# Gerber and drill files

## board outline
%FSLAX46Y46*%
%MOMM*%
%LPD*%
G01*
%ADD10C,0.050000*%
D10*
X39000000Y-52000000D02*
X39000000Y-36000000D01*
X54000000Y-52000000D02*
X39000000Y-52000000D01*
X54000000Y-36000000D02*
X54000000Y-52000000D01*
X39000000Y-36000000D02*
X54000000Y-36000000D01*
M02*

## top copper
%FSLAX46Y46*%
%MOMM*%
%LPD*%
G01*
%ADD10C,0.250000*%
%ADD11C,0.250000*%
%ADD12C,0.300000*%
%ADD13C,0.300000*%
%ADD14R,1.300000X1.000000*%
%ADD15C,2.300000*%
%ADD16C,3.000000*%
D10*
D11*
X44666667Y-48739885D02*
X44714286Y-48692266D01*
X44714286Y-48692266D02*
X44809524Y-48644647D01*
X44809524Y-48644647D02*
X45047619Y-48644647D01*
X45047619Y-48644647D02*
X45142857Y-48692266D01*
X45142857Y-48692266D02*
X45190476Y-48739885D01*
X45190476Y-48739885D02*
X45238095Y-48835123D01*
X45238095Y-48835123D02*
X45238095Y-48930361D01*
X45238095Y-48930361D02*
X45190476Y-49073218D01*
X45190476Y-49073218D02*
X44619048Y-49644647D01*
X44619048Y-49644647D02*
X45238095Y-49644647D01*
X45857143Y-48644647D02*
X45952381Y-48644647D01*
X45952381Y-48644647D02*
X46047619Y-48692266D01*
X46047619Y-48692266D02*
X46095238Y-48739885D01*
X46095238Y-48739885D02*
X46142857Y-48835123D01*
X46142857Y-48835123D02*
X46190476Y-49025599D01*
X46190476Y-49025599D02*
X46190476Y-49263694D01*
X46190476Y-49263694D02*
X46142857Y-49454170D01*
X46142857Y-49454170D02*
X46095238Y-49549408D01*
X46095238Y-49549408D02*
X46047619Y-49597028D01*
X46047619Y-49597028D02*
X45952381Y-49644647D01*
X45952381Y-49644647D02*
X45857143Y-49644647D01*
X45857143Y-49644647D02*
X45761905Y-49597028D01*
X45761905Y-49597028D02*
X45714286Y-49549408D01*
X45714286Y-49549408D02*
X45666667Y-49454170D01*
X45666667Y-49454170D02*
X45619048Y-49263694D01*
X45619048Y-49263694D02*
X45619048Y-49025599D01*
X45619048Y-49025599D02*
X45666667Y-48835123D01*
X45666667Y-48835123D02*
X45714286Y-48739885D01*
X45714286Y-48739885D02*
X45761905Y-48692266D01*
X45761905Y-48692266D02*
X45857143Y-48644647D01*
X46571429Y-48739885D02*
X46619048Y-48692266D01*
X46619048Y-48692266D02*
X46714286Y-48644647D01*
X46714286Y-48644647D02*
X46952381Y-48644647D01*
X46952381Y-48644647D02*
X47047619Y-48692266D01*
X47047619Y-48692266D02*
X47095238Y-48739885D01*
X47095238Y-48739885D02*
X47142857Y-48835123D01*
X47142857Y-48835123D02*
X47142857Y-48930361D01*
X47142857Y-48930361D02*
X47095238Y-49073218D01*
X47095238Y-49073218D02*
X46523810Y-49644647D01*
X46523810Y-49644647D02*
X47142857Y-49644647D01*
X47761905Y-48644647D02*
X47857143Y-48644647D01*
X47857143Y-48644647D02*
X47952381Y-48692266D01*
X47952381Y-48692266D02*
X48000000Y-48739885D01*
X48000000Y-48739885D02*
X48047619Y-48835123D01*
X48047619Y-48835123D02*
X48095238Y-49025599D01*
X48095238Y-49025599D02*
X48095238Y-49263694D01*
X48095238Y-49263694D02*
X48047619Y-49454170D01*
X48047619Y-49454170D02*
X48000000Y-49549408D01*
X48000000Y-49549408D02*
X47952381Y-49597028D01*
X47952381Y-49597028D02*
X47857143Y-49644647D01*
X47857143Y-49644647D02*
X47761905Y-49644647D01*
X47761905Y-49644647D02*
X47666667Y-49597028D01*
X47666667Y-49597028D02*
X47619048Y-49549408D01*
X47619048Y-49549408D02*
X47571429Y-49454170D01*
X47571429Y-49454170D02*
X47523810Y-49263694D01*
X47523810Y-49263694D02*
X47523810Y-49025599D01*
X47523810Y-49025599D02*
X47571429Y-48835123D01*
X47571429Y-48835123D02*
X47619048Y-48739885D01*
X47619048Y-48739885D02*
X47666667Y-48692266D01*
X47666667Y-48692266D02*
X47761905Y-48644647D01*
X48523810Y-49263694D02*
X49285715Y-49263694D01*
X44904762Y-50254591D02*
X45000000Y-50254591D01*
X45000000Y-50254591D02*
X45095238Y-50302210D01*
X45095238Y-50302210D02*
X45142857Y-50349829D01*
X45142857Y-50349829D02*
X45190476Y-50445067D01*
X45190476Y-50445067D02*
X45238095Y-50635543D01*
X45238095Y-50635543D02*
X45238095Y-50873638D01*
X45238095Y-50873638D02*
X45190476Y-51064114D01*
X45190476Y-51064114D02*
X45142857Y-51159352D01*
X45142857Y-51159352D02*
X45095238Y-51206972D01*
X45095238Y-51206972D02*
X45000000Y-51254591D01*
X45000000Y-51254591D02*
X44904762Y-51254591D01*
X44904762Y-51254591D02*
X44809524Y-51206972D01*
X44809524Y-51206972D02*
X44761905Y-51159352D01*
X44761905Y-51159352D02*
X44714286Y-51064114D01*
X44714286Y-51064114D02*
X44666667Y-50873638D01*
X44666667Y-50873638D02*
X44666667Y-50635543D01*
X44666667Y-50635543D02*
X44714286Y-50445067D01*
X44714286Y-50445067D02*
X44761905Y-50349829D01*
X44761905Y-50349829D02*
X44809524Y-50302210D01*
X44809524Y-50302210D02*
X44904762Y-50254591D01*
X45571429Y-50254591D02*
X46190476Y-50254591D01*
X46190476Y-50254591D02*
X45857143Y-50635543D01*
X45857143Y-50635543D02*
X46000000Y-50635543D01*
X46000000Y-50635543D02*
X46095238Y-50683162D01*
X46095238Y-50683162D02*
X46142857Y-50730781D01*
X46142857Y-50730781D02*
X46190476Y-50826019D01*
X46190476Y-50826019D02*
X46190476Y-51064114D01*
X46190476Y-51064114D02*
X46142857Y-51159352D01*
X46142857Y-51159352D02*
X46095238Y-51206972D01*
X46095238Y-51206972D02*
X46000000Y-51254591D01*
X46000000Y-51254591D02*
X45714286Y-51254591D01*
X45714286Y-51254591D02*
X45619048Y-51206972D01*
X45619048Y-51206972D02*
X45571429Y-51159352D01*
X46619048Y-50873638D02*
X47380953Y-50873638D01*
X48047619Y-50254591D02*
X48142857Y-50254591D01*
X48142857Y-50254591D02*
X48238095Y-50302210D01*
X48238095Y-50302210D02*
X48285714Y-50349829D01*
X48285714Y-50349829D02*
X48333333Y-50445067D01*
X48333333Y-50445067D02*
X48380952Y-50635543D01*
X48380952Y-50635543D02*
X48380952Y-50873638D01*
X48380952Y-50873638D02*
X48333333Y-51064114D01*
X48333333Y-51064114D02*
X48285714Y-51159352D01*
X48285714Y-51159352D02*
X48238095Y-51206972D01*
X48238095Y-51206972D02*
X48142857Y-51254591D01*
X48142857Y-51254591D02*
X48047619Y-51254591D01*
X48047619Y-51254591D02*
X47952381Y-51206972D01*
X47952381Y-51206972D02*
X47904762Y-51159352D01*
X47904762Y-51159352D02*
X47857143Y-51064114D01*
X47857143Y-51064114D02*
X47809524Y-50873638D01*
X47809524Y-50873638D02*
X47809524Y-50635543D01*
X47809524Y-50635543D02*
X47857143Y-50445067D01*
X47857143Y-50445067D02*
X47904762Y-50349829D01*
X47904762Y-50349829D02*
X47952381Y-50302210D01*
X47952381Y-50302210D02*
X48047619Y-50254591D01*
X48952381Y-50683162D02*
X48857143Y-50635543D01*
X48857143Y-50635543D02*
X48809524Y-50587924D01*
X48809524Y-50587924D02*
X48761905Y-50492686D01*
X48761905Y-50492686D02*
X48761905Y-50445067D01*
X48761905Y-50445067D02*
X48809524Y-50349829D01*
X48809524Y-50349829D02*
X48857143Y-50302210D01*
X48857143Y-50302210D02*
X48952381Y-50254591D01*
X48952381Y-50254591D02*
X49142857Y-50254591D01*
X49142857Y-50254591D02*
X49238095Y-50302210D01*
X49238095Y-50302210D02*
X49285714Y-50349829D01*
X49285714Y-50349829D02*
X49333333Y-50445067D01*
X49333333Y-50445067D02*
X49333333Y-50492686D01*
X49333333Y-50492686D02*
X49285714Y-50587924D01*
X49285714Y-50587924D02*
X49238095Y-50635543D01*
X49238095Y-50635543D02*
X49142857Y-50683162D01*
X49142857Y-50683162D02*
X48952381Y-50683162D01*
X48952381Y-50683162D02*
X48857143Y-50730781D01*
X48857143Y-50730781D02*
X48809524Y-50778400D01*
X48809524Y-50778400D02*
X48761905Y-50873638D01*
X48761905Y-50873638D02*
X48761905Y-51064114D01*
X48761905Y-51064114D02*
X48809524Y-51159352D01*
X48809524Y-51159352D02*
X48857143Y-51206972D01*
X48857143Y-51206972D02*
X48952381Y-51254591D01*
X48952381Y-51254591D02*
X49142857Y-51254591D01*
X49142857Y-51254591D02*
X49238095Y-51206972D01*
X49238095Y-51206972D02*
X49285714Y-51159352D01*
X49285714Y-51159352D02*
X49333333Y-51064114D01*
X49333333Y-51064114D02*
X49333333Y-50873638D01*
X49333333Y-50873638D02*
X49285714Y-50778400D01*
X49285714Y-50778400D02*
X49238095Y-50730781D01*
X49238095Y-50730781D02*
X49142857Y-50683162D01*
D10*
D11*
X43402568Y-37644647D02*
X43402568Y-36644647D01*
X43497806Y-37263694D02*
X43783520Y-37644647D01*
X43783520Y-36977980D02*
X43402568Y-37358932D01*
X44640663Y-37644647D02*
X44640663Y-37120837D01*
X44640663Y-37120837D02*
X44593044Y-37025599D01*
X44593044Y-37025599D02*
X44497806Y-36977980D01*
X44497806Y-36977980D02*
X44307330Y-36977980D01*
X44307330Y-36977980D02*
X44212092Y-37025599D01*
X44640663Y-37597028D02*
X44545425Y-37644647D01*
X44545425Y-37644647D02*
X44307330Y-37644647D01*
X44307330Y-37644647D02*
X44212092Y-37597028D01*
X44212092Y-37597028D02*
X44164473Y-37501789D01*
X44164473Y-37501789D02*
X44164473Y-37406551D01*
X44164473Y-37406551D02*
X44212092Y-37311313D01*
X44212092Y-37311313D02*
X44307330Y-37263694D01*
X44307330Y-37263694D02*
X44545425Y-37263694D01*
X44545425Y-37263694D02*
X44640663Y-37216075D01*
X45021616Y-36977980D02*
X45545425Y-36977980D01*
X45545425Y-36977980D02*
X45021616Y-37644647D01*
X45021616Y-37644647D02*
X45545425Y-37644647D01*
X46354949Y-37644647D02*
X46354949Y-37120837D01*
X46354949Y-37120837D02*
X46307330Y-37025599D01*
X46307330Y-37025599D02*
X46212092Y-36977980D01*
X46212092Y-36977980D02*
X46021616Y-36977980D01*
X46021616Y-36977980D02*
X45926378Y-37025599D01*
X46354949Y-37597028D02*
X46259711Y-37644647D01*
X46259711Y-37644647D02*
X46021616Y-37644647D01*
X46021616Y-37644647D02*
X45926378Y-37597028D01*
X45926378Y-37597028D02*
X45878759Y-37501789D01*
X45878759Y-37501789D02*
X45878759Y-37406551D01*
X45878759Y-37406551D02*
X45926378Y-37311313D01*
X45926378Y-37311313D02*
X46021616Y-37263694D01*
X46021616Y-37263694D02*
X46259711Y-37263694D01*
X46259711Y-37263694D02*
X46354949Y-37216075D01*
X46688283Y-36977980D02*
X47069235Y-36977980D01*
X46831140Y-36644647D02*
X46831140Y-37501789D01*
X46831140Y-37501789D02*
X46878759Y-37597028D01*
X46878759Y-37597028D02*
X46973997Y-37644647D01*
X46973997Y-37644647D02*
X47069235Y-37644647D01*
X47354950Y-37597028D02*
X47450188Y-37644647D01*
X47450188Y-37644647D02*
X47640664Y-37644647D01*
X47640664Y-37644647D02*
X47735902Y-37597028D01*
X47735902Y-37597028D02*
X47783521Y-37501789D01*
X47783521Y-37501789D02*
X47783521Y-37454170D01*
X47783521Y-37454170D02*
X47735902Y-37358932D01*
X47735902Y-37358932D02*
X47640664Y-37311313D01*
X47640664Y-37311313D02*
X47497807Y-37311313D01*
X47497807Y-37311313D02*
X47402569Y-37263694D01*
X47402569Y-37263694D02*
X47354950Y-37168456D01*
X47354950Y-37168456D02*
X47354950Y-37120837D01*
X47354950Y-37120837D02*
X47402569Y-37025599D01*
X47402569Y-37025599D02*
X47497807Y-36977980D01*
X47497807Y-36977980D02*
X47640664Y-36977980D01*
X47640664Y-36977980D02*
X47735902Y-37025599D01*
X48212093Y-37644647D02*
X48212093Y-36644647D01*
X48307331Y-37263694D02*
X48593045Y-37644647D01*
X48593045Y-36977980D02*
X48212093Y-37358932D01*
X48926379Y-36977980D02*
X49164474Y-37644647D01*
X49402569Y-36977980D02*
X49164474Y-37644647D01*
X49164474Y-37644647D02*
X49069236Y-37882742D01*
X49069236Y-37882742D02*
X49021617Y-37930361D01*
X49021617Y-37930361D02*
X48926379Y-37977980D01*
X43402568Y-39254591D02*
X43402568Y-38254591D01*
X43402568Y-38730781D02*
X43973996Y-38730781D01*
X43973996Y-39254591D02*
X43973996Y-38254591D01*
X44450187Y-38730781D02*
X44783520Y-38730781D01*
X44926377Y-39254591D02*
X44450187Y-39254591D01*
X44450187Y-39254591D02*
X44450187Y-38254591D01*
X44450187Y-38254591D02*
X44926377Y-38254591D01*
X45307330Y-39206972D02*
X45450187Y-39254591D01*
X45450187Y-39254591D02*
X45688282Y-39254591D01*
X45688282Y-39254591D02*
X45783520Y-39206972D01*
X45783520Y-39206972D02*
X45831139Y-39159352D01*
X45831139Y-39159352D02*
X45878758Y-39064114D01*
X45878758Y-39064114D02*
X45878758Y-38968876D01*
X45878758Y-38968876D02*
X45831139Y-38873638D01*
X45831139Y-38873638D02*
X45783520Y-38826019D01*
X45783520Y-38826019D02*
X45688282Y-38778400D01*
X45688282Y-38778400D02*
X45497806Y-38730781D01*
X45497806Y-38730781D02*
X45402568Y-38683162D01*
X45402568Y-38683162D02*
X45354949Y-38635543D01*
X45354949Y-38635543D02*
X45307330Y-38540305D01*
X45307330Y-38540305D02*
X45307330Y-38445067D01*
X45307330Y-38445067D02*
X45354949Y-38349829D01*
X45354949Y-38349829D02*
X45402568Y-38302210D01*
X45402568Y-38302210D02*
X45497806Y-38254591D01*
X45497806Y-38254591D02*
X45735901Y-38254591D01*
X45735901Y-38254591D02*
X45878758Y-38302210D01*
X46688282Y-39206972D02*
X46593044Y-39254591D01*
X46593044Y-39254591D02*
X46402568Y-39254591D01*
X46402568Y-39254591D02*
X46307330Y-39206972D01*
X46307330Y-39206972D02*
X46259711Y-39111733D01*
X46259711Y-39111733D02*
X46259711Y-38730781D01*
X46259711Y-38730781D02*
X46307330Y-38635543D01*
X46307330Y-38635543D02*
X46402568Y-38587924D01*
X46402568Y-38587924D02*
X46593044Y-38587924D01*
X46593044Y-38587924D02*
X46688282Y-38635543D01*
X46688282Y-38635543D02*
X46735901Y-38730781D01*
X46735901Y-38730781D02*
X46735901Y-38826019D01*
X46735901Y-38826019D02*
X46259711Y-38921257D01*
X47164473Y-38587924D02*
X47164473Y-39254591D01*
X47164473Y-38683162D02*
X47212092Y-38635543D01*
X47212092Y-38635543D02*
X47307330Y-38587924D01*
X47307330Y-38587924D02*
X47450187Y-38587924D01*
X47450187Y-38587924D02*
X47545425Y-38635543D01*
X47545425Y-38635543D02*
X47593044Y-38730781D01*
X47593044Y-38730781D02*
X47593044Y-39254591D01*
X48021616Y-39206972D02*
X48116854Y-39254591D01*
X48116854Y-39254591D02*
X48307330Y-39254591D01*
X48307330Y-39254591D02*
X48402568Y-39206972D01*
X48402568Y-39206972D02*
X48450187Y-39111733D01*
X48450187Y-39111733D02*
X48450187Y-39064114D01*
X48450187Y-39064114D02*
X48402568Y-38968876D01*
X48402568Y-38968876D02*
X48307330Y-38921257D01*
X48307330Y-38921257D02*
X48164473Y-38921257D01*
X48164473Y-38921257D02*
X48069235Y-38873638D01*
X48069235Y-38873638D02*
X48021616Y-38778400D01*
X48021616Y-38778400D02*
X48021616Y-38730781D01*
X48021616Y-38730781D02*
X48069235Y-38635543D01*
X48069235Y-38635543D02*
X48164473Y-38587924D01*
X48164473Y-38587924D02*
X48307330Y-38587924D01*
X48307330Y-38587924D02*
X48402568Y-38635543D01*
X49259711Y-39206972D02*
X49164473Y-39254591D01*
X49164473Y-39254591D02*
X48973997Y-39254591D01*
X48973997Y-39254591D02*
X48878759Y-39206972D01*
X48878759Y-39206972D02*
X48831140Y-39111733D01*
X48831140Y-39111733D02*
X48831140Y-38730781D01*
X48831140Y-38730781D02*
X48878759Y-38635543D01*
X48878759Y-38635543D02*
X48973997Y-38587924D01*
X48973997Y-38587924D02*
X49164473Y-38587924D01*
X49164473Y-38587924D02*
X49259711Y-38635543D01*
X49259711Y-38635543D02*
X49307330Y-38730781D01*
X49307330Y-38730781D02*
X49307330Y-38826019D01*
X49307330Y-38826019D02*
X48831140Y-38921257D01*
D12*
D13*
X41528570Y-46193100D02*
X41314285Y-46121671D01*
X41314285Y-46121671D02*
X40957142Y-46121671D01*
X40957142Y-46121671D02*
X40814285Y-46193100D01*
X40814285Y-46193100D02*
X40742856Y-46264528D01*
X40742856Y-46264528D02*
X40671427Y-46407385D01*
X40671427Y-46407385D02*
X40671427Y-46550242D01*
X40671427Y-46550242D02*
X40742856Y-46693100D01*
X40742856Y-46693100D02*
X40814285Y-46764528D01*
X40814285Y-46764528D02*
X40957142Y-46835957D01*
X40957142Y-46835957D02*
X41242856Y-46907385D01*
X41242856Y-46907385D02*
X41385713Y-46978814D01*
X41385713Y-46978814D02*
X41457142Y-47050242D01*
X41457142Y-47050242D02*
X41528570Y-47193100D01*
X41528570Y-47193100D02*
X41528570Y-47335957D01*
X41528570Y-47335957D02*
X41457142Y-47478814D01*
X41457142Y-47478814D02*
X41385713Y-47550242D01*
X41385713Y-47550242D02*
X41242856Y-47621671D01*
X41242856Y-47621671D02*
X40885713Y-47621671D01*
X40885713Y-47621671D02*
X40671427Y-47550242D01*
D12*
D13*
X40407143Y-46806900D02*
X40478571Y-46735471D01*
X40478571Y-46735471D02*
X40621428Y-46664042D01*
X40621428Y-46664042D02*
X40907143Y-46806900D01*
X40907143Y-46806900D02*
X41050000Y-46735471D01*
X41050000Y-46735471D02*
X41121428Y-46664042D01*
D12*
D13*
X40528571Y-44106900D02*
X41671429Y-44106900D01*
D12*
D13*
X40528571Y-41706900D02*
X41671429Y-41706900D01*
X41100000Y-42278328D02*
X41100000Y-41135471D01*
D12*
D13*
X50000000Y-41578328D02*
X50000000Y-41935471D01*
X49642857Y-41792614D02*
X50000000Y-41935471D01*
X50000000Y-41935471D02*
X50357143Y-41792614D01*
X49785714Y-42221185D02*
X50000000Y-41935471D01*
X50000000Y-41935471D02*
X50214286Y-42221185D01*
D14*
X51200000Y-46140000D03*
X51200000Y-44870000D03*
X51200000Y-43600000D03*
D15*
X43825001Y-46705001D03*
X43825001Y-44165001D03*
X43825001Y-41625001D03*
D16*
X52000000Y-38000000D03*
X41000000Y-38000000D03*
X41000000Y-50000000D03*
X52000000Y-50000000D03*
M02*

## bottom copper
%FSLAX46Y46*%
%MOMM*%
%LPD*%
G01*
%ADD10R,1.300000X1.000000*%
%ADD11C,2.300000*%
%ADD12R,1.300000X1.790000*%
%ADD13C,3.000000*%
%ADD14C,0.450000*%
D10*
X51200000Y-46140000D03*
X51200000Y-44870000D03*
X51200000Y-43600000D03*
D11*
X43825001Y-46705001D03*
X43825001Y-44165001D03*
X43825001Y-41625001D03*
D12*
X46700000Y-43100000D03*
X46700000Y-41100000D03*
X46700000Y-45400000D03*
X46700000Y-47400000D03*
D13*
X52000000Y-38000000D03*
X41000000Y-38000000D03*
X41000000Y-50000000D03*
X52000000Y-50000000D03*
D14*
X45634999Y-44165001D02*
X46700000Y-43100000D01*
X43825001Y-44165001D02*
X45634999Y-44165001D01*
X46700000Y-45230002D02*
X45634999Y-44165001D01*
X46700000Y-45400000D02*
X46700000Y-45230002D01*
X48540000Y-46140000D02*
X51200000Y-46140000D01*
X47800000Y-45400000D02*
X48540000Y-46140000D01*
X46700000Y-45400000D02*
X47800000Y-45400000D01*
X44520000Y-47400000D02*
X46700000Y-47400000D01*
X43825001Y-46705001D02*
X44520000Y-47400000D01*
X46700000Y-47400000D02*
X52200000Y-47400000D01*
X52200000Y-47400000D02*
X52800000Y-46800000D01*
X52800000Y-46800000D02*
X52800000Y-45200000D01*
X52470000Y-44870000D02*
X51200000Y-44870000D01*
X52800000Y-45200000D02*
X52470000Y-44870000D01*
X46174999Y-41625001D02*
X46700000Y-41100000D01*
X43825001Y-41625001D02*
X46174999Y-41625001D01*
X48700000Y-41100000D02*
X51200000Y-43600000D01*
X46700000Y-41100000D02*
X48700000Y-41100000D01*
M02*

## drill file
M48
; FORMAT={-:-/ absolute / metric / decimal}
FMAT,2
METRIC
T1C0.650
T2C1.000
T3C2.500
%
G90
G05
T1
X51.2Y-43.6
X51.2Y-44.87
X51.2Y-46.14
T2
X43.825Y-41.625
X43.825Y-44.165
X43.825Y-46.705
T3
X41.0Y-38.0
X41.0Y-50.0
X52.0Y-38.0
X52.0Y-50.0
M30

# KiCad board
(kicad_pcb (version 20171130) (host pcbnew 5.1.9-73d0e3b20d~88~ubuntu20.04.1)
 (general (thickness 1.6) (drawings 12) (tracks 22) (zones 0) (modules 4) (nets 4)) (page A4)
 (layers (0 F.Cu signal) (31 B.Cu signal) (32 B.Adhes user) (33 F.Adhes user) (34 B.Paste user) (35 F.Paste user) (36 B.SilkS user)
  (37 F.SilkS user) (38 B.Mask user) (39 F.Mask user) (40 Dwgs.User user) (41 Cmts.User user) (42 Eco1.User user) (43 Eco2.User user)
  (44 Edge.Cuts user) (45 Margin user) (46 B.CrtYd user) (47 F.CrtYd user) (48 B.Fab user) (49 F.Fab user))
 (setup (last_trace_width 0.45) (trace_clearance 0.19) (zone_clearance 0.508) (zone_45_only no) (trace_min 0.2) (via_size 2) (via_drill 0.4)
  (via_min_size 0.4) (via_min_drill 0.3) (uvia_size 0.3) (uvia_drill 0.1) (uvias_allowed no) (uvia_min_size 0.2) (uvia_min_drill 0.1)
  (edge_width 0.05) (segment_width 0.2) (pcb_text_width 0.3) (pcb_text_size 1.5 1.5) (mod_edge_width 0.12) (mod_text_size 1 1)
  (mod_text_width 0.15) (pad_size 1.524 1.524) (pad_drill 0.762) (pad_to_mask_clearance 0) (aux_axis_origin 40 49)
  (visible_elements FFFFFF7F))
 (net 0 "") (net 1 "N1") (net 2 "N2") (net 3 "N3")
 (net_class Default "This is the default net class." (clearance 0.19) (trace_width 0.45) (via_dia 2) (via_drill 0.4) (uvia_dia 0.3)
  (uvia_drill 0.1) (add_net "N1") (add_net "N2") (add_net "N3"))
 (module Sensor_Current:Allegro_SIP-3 (layer F.Cu) (at 51.2 43.6 270)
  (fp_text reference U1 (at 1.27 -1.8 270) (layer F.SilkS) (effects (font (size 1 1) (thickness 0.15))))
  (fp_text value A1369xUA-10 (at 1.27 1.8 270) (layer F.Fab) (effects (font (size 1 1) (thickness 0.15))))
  (pad 3 thru_hole rect (at 2.54 0 270) (size 1 1.3) (drill 0.65) (layers *.Cu *.Mask) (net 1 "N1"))
  (pad 2 thru_hole rect (at 1.27 0 270) (size 1 1.3) (drill 0.65) (layers *.Cu *.Mask) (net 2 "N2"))
  (pad 1 thru_hole rect (at 0 0 270) (size 1 1.3) (drill 0.65) (layers *.Cu *.Mask) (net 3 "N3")))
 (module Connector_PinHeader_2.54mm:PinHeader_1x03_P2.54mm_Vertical (layer F.Cu) (at 43.825001 41.625001)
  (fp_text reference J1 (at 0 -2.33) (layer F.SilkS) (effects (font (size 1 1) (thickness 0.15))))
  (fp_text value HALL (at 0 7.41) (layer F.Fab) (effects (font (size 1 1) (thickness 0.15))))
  (pad 3 thru_hole circle (at 0 5.08) (size 2.3 2.3) (drill 1) (layers *.Cu *.Mask) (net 2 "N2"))
  (pad 2 thru_hole circle (at 0 2.54) (size 2.3 2.3) (drill 1) (layers *.Cu *.Mask) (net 1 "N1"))
  (pad 1 thru_hole circle (at 0 0) (size 2.3 2.3) (drill 1) (layers *.Cu *.Mask) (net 3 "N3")))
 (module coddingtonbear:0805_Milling (layer B.Cu) (at 46.7 42.1 90)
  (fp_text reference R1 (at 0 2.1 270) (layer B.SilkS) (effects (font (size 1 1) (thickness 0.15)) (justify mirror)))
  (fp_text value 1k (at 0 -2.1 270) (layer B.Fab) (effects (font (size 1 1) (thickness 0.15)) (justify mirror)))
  (pad 1 smd rect (at -1 0 90) (size 1.79 1.3) (layers B.Cu B.Paste B.Mask) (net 1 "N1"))
  (pad 2 smd rect (at 1 0 90) (size 1.79 1.3) (layers B.Cu B.Paste B.Mask) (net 3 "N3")))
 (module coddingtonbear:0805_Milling (layer B.Cu) (at 46.7 46.4 270)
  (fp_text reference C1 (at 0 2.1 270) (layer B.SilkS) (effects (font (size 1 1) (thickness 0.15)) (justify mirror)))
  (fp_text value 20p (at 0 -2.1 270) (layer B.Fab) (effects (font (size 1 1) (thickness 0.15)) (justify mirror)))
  (pad 1 smd rect (at -1 0 270) (size 1.79 1.3) (layers B.Cu B.Paste B.Mask) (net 1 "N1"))
  (pad 2 smd rect (at 1 0 270) (size 1.79 1.3) (layers B.Cu B.Paste B.Mask) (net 2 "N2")))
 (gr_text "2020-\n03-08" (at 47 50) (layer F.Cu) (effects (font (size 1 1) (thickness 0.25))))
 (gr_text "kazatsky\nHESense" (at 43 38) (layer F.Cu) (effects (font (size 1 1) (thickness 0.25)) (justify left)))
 (gr_line (start 39 52) (end 39 36) (layer Edge.Cuts) (width 0.05))
 (gr_line (start 54 52) (end 39 52) (layer Edge.Cuts) (width 0.05))
 (gr_line (start 54 36) (end 54 52) (layer Edge.Cuts) (width 0.05))
 (gr_line (start 39 36) (end 54 36) (layer Edge.Cuts) (width 0.05))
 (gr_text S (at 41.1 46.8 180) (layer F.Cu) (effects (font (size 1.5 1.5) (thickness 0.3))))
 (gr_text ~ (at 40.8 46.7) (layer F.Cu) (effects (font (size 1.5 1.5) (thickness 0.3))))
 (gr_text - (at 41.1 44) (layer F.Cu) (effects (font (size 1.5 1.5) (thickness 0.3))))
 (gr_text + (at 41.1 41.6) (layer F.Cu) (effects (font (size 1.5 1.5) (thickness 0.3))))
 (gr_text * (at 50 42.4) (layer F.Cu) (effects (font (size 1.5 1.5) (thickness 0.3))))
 (via (at 52 38) (size 3) (drill 2.5) (layers F.Cu B.Cu) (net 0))
 (via (at 41 38) (size 3) (drill 2.5) (layers F.Cu B.Cu) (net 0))
 (via (at 41 50) (size 3) (drill 2.5) (layers F.Cu B.Cu) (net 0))
 (via (at 52 50) (size 3) (drill 2.5) (layers F.Cu B.Cu) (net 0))
 (segment (start 45.634999 44.165001) (end 46.7 43.1) (width 0.45) (layer B.Cu) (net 1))
 (segment (start 43.825001 44.165001) (end 45.634999 44.165001) (width 0.45) (layer B.Cu) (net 1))
 (segment (start 46.7 45.230002) (end 45.634999 44.165001) (width 0.45) (layer B.Cu) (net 1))
 (segment (start 46.7 45.4) (end 46.7 45.230002) (width 0.45) (layer B.Cu) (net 1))
 (segment (start 48.54 46.14) (end 51.2 46.14) (width 0.45) (layer B.Cu) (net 1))
 (segment (start 47.8 45.4) (end 48.54 46.14) (width 0.45) (layer B.Cu) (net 1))
 (segment (start 46.7 45.4) (end 47.8 45.4) (width 0.45) (layer B.Cu) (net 1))
 (segment (start 44.52 47.4) (end 46.7 47.4) (width 0.45) (layer B.Cu) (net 2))
 (segment (start 43.825001 46.705001) (end 44.52 47.4) (width 0.45) (layer B.Cu) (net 2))
 (segment (start 46.7 47.4) (end 52.2 47.4) (width 0.45) (layer B.Cu) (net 2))
 (segment (start 52.2 47.4) (end 52.8 46.8) (width 0.45) (layer B.Cu) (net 2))
 (segment (start 52.8 46.8) (end 52.8 45.2) (width 0.45) (layer B.Cu) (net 2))
 (segment (start 52.47 44.87) (end 51.2 44.87) (width 0.45) (layer B.Cu) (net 2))
 (segment (start 52.8 45.2) (end 52.47 44.87) (width 0.45) (layer B.Cu) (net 2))
 (segment (start 46.174999 41.625001) (end 46.7 41.1) (width 0.45) (layer B.Cu) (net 3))
 (segment (start 43.825001 41.625001) (end 46.174999 41.625001) (width 0.45) (layer B.Cu) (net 3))
 (segment (start 48.7 41.1) (end 51.2 43.6) (width 0.45) (layer B.Cu) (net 3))
 (segment (start 46.7 41.1) (end 48.7 41.1) (width 0.45) (layer B.Cu) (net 3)))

